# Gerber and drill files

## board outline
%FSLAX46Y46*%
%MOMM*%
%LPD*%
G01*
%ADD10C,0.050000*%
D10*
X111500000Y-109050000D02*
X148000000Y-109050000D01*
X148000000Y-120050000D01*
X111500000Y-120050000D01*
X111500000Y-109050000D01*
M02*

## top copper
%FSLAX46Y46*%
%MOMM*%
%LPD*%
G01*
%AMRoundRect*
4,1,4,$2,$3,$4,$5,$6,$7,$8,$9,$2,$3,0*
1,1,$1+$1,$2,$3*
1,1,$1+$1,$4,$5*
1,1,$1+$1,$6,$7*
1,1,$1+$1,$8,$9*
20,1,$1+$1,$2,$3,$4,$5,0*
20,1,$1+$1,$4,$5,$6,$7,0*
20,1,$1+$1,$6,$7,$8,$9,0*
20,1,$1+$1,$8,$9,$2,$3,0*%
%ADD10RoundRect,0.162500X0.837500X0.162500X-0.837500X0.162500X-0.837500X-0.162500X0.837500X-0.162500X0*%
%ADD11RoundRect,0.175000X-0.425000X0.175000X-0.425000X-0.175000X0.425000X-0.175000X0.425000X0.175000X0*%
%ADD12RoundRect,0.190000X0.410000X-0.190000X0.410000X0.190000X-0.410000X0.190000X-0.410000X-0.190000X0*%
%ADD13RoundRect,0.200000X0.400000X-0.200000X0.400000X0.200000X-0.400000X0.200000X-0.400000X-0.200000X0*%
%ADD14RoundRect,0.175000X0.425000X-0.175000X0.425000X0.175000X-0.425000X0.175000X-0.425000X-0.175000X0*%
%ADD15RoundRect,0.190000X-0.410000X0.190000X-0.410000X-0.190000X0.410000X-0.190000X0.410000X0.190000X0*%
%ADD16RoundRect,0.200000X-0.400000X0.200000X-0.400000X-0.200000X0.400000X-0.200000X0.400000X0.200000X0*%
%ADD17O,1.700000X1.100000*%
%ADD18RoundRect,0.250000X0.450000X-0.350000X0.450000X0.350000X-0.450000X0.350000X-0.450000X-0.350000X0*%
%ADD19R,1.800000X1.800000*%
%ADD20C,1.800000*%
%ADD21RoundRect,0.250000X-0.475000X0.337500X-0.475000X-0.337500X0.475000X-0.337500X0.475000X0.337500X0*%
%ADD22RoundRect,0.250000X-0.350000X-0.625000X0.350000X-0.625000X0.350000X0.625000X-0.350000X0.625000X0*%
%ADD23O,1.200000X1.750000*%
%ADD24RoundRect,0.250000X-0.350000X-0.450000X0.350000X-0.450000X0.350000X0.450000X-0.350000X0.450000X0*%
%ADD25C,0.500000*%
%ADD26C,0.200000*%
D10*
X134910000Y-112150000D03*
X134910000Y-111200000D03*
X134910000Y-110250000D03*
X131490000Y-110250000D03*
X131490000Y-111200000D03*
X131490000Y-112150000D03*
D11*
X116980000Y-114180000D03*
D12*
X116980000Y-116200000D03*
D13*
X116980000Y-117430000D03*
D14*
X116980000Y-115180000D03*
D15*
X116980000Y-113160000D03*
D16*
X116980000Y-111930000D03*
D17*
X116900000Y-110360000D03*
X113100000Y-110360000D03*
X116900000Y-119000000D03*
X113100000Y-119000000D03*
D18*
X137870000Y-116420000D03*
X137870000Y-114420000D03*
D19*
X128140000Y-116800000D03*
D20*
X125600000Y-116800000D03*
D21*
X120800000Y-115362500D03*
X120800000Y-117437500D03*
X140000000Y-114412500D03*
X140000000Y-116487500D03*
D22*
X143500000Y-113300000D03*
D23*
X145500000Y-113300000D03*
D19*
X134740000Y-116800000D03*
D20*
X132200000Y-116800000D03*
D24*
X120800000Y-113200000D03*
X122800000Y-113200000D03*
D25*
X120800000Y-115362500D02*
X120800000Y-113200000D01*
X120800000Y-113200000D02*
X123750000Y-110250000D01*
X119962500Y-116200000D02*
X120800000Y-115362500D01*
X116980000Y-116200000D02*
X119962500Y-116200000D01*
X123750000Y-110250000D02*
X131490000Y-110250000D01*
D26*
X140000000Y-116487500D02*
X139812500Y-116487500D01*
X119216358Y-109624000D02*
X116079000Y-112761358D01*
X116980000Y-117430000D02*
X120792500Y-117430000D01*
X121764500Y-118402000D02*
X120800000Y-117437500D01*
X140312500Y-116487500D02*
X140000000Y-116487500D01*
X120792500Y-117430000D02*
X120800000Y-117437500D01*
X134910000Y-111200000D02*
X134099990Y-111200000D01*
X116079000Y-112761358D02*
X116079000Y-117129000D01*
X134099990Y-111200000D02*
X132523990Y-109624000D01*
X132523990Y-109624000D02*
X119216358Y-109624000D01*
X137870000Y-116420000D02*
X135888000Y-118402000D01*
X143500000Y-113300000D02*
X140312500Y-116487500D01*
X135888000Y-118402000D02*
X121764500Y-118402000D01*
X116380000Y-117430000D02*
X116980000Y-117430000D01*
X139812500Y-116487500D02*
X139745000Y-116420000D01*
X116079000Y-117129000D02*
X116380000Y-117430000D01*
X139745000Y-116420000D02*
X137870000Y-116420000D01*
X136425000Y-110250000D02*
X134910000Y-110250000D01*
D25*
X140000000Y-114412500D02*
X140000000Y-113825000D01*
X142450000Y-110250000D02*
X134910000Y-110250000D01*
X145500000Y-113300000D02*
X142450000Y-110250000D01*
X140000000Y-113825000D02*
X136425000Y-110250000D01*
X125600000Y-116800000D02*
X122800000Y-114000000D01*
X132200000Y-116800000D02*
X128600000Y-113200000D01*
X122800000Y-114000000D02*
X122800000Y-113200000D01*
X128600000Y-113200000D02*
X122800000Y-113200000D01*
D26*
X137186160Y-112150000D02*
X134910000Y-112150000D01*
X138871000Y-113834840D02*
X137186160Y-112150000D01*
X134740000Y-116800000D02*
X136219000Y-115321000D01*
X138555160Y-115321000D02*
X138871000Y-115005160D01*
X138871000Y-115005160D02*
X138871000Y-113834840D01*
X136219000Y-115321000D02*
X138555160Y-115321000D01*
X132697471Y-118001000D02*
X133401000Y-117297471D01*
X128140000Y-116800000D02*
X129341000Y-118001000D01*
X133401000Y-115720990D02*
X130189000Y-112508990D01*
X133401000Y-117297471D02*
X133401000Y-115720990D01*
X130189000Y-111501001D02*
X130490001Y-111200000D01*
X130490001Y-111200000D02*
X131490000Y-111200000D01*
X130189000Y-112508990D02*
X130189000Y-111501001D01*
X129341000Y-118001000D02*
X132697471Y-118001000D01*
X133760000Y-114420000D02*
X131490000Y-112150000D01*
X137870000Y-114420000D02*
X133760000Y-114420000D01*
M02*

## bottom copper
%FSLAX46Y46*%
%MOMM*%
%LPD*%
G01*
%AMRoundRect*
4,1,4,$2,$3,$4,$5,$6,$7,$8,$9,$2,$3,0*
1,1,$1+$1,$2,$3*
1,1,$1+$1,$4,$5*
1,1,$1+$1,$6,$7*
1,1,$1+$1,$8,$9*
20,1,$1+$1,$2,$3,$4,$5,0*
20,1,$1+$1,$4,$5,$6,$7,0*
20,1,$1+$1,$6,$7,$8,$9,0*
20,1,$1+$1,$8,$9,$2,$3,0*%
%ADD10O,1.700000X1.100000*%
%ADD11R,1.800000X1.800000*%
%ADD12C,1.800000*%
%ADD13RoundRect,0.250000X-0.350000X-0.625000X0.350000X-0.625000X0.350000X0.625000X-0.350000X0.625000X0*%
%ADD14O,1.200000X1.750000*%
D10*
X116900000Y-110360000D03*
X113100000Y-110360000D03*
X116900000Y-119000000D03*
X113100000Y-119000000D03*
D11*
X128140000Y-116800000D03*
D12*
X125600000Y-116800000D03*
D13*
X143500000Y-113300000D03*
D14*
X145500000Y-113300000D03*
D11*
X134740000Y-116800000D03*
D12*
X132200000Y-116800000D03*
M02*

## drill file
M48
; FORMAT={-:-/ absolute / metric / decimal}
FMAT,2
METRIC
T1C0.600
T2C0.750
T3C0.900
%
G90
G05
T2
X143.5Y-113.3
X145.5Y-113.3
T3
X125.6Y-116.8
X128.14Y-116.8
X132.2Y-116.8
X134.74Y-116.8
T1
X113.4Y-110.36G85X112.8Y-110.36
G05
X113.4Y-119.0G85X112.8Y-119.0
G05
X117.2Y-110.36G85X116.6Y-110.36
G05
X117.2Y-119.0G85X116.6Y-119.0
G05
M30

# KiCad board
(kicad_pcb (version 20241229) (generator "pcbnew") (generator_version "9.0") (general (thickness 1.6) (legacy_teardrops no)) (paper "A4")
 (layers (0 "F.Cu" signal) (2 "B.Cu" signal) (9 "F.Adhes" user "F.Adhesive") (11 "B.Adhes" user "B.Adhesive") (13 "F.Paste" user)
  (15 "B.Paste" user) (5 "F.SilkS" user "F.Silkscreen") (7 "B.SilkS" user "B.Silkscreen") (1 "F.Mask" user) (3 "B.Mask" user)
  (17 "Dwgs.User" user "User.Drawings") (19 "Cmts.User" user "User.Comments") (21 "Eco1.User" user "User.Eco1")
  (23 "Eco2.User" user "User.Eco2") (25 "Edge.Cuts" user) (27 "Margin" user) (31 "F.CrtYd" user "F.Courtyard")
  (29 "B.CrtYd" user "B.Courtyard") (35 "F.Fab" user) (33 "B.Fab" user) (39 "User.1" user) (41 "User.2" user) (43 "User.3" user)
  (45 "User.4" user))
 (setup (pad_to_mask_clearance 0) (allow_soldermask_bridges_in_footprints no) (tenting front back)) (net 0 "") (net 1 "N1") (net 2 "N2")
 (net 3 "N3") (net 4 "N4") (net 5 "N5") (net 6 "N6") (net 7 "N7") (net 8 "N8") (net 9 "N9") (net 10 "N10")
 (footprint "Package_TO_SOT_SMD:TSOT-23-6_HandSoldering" (layer "F.Cu") (at 133.2 111.2 180)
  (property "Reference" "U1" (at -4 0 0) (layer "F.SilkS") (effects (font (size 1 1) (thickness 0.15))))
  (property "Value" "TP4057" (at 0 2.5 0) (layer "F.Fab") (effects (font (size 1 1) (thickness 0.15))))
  (pad "1" smd roundrect (at -1.71 -0.95 180) (size 2 0.65) (layers "F.Cu" "F.Mask" "F.Paste") (roundrect_rratio 0.25) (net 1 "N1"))
  (pad "2" smd roundrect (at -1.71 0 180) (size 2 0.65) (layers "F.Cu" "F.Mask" "F.Paste") (roundrect_rratio 0.25) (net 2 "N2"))
  (pad "3" smd roundrect (at -1.71 0.95 180) (size 2 0.65) (layers "F.Cu" "F.Mask" "F.Paste") (roundrect_rratio 0.25) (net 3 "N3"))
  (pad "4" smd roundrect (at 1.71 0.95 180) (size 2 0.65) (layers "F.Cu" "F.Mask" "F.Paste") (roundrect_rratio 0.25) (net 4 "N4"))
  (pad "5" smd roundrect (at 1.71 0 180) (size 2 0.65) (layers "F.Cu" "F.Mask" "F.Paste") (roundrect_rratio 0.25) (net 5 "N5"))
  (pad "6" smd roundrect (at 1.71 -0.95 180) (size 2 0.65) (layers "F.Cu" "F.Mask" "F.Paste") (roundrect_rratio 0.25) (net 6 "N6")))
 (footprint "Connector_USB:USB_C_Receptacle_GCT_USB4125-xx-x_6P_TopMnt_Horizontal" (layer "F.Cu") (at 113.9 114.68 -90)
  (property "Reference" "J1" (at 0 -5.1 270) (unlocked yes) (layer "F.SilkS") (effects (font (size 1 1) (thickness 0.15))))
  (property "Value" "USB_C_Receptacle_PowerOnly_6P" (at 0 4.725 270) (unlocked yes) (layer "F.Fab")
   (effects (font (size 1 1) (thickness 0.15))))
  (pad "A5" smd roundrect (at -0.5 -3.08 270) (size 0.7 1.2) (layers "F.Cu" "F.Mask" "F.Paste") (roundrect_rratio 0.25) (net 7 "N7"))
  (pad "A9" smd roundrect (at 1.52 -3.08 90) (size 0.76 1.2) (layers "F.Cu" "F.Mask" "F.Paste") (roundrect_rratio 0.25) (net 4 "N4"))
  (pad "A12" smd roundrect (at 2.75 -3.08 90) (size 0.8 1.2) (layers "F.Cu" "F.Mask" "F.Paste") (roundrect_rratio 0.25) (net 2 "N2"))
  (pad "B5" smd roundrect (at 0.5 -3.08 90) (size 0.7 1.2) (layers "F.Cu" "F.Mask" "F.Paste") (roundrect_rratio 0.25) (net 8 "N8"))
  (pad "B9" smd roundrect (at -1.52 -3.08 270) (size 0.76 1.2) (layers "F.Cu" "F.Mask" "F.Paste") (roundrect_rratio 0.25) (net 4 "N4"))
  (pad "B12" smd roundrect (at -2.75 -3.08 270) (size 0.8 1.2) (layers "F.Cu" "F.Mask" "F.Paste") (roundrect_rratio 0.25) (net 2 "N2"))
  (pad "S1" thru_hole oval (at -4.32 -3 270) (size 1.1 1.7) (drill oval 0.6 1.2) (layers "*.Cu" "*.Mask" "F.Paste")
   (remove_unused_layers no) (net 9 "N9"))
  (pad "S1" thru_hole oval (at -4.32 0.8 270) (size 1.1 1.7) (drill oval 0.6 1.2) (layers "*.Cu" "*.Mask" "F.Paste")
   (remove_unused_layers no) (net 9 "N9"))
  (pad "S1" thru_hole oval (at 4.32 -3 270) (size 1.1 1.7) (drill oval 0.6 1.2) (layers "*.Cu" "*.Mask" "F.Paste") (remove_unused_layers no)
   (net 9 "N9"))
  (pad "S1" thru_hole oval (at 4.32 0.8 270) (size 1.1 1.7) (drill oval 0.6 1.2) (layers "*.Cu" "*.Mask" "F.Paste")
   (remove_unused_layers no) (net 9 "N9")))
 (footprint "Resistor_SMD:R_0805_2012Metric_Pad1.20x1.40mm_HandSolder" (layer "F.Cu") (at 137.87 115.42 90)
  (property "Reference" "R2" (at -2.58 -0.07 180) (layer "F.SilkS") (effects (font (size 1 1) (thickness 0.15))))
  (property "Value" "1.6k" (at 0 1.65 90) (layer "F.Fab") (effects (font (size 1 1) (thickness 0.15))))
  (pad "1" smd roundrect (at -1 0 90) (size 1.2 1.4) (layers "F.Cu" "F.Mask" "F.Paste") (roundrect_rratio 0.208333) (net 2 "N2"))
  (pad "2" smd roundrect (at 1 0 90) (size 1.2 1.4) (layers "F.Cu" "F.Mask" "F.Paste") (roundrect_rratio 0.208333) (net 6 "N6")))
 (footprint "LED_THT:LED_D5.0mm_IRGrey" (layer "F.Cu") (at 128.14 116.8 180)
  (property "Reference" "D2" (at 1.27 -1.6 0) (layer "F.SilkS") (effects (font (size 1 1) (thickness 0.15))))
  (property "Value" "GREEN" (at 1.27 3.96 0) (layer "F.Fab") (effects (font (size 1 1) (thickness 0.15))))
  (pad "1" thru_hole rect (at 0 0 180) (size 1.8 1.8) (drill 0.9) (layers "*.Cu" "*.Mask") (remove_unused_layers no) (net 5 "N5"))
  (pad "2" thru_hole circle (at 2.54 0 180) (size 1.8 1.8) (drill 0.9) (layers "*.Cu" "*.Mask") (remove_unused_layers no) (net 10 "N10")))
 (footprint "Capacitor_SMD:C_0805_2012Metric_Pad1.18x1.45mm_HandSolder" (layer "F.Cu") (at 120.8 116.4 -90)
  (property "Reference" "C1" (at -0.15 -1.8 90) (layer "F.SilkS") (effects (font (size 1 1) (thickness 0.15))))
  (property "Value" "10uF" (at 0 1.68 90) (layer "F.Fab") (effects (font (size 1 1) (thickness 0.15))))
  (pad "1" smd roundrect (at -1.0375 0 270) (size 1.175 1.45) (layers "F.Cu" "F.Mask" "F.Paste") (roundrect_rratio 0.212766) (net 4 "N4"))
  (pad "2" smd roundrect (at 1.0375 0 270) (size 1.175 1.45) (layers "F.Cu" "F.Mask" "F.Paste") (roundrect_rratio 0.212766) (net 2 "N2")))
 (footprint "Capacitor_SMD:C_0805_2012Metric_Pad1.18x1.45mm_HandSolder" (layer "F.Cu") (at 140 115.45 -90)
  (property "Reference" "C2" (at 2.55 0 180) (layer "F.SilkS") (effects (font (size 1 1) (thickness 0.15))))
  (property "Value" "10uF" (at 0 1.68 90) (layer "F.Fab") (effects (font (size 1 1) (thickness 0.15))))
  (pad "1" smd roundrect (at -1.0375 0 270) (size 1.175 1.45) (layers "F.Cu" "F.Mask" "F.Paste") (roundrect_rratio 0.212766) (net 3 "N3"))
  (pad "2" smd roundrect (at 1.0375 0 270) (size 1.175 1.45) (layers "F.Cu" "F.Mask" "F.Paste") (roundrect_rratio 0.212766) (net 2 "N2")))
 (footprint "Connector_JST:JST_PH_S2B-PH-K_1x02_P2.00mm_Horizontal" (layer "F.Cu") (at 143.5 113.3)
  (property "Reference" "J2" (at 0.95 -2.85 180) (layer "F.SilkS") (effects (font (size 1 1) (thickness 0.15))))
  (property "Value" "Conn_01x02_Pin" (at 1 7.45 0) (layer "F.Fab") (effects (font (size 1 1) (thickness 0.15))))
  (pad "1" thru_hole roundrect (at 0 0) (size 1.2 1.75) (drill 0.75) (layers "*.Cu" "*.Mask") (remove_unused_layers no)
   (roundrect_rratio 0.208333) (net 2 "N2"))
  (pad "2" thru_hole oval (at 2 0) (size 1.2 1.75) (drill 0.75) (layers "*.Cu" "*.Mask") (remove_unused_layers no) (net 3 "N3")))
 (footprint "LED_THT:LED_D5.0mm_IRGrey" (layer "F.Cu") (at 134.74 116.8 180)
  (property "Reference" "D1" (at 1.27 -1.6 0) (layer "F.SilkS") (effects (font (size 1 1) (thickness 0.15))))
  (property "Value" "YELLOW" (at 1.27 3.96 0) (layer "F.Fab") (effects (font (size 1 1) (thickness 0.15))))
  (pad "1" thru_hole rect (at 0 0 180) (size 1.8 1.8) (drill 0.9) (layers "*.Cu" "*.Mask") (remove_unused_layers no) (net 1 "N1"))
  (pad "2" thru_hole circle (at 2.54 0 180) (size 1.8 1.8) (drill 0.9) (layers "*.Cu" "*.Mask") (remove_unused_layers no) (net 10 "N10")))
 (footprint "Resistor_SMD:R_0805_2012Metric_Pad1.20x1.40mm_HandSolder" (layer "F.Cu") (at 121.8 113.2)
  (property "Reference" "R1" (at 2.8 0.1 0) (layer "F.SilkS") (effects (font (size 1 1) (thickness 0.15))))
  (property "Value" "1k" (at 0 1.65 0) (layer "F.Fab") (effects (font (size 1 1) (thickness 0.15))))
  (pad "1" smd roundrect (at -1 0) (size 1.2 1.4) (layers "F.Cu" "F.Mask" "F.Paste") (roundrect_rratio 0.208333) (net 4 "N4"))
  (pad "2" smd roundrect (at 1 0) (size 1.2 1.4) (layers "F.Cu" "F.Mask" "F.Paste") (roundrect_rratio 0.208333) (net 10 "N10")))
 (gr_rect (start 111.5 109.05) (end 148 120.05) (stroke (width 0.05) (type solid)) (fill no) (layer "Edge.Cuts"))
 (segment (start 120.8 115.3625) (end 120.8 113.2) (width 0.5) (layer "F.Cu") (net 4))
 (segment (start 120.8 113.2) (end 123.75 110.25) (width 0.5) (layer "F.Cu") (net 4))
 (segment (start 119.9625 116.2) (end 120.8 115.3625) (width 0.5) (layer "F.Cu") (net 4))
 (segment (start 116.98 116.2) (end 119.9625 116.2) (width 0.5) (layer "F.Cu") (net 4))
 (segment (start 123.75 110.25) (end 131.49 110.25) (width 0.5) (layer "F.Cu") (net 4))
 (segment (start 140 116.4875) (end 139.8125 116.4875) (width 0.2) (layer "F.Cu") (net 2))
 (segment (start 119.216358 109.624) (end 116.079 112.761358) (width 0.2) (layer "F.Cu") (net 2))
 (segment (start 116.98 117.43) (end 120.7925 117.43) (width 0.2) (layer "F.Cu") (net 2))
 (segment (start 121.7645 118.402) (end 120.8 117.4375) (width 0.2) (layer "F.Cu") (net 2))
 (segment (start 140.3125 116.4875) (end 140 116.4875) (width 0.2) (layer "F.Cu") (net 2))
 (segment (start 120.7925 117.43) (end 120.8 117.4375) (width 0.2) (layer "F.Cu") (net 2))
 (segment (start 134.91 111.2) (end 134.09999 111.2) (width 0.2) (layer "F.Cu") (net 2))
 (segment (start 116.079 112.761358) (end 116.079 117.129) (width 0.2) (layer "F.Cu") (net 2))
 (segment (start 134.09999 111.2) (end 132.52399 109.624) (width 0.2) (layer "F.Cu") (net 2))
 (segment (start 132.52399 109.624) (end 119.216358 109.624) (width 0.2) (layer "F.Cu") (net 2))
 (segment (start 137.87 116.42) (end 135.888 118.402) (width 0.2) (layer "F.Cu") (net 2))
 (segment (start 143.5 113.3) (end 140.3125 116.4875) (width 0.2) (layer "F.Cu") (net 2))
 (segment (start 135.888 118.402) (end 121.7645 118.402) (width 0.2) (layer "F.Cu") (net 2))
 (segment (start 116.38 117.43) (end 116.98 117.43) (width 0.2) (layer "F.Cu") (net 2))
 (segment (start 139.8125 116.4875) (end 139.745 116.42) (width 0.2) (layer "F.Cu") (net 2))
 (segment (start 116.079 117.129) (end 116.38 117.43) (width 0.2) (layer "F.Cu") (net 2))
 (segment (start 139.745 116.42) (end 137.87 116.42) (width 0.2) (layer "F.Cu") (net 2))
 (segment (start 136.425 110.25) (end 134.91 110.25) (width 0.2) (layer "F.Cu") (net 3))
 (segment (start 140 114.4125) (end 140 113.825) (width 0.5) (layer "F.Cu") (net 3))
 (segment (start 142.45 110.25) (end 134.91 110.25) (width 0.5) (layer "F.Cu") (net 3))
 (segment (start 145.5 113.3) (end 142.45 110.25) (width 0.5) (layer "F.Cu") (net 3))
 (segment (start 140 113.825) (end 136.425 110.25) (width 0.5) (layer "F.Cu") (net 3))
 (segment (start 125.6 116.8) (end 122.8 114) (width 0.5) (layer "F.Cu") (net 10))
 (segment (start 132.2 116.8) (end 128.6 113.2) (width 0.5) (layer "F.Cu") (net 10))
 (segment (start 122.8 114) (end 122.8 113.2) (width 0.5) (layer "F.Cu") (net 10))
 (segment (start 128.6 113.2) (end 122.8 113.2) (width 0.5) (layer "F.Cu") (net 10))
 (segment (start 137.18616 112.15) (end 134.91 112.15) (width 0.2) (layer "F.Cu") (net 1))
 (segment (start 138.871 113.83484) (end 137.18616 112.15) (width 0.2) (layer "F.Cu") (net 1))
 (segment (start 134.74 116.8) (end 136.219 115.321) (width 0.2) (layer "F.Cu") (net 1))
 (segment (start 138.55516 115.321) (end 138.871 115.00516) (width 0.2) (layer "F.Cu") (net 1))
 (segment (start 138.871 115.00516) (end 138.871 113.83484) (width 0.2) (layer "F.Cu") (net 1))
 (segment (start 136.219 115.321) (end 138.55516 115.321) (width 0.2) (layer "F.Cu") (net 1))
 (segment (start 132.697471 118.001) (end 133.401 117.297471) (width 0.2) (layer "F.Cu") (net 5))
 (segment (start 128.14 116.8) (end 129.341 118.001) (width 0.2) (layer "F.Cu") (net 5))
 (segment (start 133.401 115.72099) (end 130.189 112.50899) (width 0.2) (layer "F.Cu") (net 5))
 (segment (start 133.401 117.297471) (end 133.401 115.72099) (width 0.2) (layer "F.Cu") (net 5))
 (segment (start 130.189 111.501001) (end 130.490001 111.2) (width 0.2) (layer "F.Cu") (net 5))
 (segment (start 130.490001 111.2) (end 131.49 111.2) (width 0.2) (layer "F.Cu") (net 5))
 (segment (start 130.189 112.50899) (end 130.189 111.501001) (width 0.2) (layer "F.Cu") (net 5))
 (segment (start 129.341 118.001) (end 132.697471 118.001) (width 0.2) (layer "F.Cu") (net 5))
 (segment (start 133.76 114.42) (end 131.49 112.15) (width 0.2) (layer "F.Cu") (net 6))
 (segment (start 137.87 114.42) (end 133.76 114.42) (width 0.2) (layer "F.Cu") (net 6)))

